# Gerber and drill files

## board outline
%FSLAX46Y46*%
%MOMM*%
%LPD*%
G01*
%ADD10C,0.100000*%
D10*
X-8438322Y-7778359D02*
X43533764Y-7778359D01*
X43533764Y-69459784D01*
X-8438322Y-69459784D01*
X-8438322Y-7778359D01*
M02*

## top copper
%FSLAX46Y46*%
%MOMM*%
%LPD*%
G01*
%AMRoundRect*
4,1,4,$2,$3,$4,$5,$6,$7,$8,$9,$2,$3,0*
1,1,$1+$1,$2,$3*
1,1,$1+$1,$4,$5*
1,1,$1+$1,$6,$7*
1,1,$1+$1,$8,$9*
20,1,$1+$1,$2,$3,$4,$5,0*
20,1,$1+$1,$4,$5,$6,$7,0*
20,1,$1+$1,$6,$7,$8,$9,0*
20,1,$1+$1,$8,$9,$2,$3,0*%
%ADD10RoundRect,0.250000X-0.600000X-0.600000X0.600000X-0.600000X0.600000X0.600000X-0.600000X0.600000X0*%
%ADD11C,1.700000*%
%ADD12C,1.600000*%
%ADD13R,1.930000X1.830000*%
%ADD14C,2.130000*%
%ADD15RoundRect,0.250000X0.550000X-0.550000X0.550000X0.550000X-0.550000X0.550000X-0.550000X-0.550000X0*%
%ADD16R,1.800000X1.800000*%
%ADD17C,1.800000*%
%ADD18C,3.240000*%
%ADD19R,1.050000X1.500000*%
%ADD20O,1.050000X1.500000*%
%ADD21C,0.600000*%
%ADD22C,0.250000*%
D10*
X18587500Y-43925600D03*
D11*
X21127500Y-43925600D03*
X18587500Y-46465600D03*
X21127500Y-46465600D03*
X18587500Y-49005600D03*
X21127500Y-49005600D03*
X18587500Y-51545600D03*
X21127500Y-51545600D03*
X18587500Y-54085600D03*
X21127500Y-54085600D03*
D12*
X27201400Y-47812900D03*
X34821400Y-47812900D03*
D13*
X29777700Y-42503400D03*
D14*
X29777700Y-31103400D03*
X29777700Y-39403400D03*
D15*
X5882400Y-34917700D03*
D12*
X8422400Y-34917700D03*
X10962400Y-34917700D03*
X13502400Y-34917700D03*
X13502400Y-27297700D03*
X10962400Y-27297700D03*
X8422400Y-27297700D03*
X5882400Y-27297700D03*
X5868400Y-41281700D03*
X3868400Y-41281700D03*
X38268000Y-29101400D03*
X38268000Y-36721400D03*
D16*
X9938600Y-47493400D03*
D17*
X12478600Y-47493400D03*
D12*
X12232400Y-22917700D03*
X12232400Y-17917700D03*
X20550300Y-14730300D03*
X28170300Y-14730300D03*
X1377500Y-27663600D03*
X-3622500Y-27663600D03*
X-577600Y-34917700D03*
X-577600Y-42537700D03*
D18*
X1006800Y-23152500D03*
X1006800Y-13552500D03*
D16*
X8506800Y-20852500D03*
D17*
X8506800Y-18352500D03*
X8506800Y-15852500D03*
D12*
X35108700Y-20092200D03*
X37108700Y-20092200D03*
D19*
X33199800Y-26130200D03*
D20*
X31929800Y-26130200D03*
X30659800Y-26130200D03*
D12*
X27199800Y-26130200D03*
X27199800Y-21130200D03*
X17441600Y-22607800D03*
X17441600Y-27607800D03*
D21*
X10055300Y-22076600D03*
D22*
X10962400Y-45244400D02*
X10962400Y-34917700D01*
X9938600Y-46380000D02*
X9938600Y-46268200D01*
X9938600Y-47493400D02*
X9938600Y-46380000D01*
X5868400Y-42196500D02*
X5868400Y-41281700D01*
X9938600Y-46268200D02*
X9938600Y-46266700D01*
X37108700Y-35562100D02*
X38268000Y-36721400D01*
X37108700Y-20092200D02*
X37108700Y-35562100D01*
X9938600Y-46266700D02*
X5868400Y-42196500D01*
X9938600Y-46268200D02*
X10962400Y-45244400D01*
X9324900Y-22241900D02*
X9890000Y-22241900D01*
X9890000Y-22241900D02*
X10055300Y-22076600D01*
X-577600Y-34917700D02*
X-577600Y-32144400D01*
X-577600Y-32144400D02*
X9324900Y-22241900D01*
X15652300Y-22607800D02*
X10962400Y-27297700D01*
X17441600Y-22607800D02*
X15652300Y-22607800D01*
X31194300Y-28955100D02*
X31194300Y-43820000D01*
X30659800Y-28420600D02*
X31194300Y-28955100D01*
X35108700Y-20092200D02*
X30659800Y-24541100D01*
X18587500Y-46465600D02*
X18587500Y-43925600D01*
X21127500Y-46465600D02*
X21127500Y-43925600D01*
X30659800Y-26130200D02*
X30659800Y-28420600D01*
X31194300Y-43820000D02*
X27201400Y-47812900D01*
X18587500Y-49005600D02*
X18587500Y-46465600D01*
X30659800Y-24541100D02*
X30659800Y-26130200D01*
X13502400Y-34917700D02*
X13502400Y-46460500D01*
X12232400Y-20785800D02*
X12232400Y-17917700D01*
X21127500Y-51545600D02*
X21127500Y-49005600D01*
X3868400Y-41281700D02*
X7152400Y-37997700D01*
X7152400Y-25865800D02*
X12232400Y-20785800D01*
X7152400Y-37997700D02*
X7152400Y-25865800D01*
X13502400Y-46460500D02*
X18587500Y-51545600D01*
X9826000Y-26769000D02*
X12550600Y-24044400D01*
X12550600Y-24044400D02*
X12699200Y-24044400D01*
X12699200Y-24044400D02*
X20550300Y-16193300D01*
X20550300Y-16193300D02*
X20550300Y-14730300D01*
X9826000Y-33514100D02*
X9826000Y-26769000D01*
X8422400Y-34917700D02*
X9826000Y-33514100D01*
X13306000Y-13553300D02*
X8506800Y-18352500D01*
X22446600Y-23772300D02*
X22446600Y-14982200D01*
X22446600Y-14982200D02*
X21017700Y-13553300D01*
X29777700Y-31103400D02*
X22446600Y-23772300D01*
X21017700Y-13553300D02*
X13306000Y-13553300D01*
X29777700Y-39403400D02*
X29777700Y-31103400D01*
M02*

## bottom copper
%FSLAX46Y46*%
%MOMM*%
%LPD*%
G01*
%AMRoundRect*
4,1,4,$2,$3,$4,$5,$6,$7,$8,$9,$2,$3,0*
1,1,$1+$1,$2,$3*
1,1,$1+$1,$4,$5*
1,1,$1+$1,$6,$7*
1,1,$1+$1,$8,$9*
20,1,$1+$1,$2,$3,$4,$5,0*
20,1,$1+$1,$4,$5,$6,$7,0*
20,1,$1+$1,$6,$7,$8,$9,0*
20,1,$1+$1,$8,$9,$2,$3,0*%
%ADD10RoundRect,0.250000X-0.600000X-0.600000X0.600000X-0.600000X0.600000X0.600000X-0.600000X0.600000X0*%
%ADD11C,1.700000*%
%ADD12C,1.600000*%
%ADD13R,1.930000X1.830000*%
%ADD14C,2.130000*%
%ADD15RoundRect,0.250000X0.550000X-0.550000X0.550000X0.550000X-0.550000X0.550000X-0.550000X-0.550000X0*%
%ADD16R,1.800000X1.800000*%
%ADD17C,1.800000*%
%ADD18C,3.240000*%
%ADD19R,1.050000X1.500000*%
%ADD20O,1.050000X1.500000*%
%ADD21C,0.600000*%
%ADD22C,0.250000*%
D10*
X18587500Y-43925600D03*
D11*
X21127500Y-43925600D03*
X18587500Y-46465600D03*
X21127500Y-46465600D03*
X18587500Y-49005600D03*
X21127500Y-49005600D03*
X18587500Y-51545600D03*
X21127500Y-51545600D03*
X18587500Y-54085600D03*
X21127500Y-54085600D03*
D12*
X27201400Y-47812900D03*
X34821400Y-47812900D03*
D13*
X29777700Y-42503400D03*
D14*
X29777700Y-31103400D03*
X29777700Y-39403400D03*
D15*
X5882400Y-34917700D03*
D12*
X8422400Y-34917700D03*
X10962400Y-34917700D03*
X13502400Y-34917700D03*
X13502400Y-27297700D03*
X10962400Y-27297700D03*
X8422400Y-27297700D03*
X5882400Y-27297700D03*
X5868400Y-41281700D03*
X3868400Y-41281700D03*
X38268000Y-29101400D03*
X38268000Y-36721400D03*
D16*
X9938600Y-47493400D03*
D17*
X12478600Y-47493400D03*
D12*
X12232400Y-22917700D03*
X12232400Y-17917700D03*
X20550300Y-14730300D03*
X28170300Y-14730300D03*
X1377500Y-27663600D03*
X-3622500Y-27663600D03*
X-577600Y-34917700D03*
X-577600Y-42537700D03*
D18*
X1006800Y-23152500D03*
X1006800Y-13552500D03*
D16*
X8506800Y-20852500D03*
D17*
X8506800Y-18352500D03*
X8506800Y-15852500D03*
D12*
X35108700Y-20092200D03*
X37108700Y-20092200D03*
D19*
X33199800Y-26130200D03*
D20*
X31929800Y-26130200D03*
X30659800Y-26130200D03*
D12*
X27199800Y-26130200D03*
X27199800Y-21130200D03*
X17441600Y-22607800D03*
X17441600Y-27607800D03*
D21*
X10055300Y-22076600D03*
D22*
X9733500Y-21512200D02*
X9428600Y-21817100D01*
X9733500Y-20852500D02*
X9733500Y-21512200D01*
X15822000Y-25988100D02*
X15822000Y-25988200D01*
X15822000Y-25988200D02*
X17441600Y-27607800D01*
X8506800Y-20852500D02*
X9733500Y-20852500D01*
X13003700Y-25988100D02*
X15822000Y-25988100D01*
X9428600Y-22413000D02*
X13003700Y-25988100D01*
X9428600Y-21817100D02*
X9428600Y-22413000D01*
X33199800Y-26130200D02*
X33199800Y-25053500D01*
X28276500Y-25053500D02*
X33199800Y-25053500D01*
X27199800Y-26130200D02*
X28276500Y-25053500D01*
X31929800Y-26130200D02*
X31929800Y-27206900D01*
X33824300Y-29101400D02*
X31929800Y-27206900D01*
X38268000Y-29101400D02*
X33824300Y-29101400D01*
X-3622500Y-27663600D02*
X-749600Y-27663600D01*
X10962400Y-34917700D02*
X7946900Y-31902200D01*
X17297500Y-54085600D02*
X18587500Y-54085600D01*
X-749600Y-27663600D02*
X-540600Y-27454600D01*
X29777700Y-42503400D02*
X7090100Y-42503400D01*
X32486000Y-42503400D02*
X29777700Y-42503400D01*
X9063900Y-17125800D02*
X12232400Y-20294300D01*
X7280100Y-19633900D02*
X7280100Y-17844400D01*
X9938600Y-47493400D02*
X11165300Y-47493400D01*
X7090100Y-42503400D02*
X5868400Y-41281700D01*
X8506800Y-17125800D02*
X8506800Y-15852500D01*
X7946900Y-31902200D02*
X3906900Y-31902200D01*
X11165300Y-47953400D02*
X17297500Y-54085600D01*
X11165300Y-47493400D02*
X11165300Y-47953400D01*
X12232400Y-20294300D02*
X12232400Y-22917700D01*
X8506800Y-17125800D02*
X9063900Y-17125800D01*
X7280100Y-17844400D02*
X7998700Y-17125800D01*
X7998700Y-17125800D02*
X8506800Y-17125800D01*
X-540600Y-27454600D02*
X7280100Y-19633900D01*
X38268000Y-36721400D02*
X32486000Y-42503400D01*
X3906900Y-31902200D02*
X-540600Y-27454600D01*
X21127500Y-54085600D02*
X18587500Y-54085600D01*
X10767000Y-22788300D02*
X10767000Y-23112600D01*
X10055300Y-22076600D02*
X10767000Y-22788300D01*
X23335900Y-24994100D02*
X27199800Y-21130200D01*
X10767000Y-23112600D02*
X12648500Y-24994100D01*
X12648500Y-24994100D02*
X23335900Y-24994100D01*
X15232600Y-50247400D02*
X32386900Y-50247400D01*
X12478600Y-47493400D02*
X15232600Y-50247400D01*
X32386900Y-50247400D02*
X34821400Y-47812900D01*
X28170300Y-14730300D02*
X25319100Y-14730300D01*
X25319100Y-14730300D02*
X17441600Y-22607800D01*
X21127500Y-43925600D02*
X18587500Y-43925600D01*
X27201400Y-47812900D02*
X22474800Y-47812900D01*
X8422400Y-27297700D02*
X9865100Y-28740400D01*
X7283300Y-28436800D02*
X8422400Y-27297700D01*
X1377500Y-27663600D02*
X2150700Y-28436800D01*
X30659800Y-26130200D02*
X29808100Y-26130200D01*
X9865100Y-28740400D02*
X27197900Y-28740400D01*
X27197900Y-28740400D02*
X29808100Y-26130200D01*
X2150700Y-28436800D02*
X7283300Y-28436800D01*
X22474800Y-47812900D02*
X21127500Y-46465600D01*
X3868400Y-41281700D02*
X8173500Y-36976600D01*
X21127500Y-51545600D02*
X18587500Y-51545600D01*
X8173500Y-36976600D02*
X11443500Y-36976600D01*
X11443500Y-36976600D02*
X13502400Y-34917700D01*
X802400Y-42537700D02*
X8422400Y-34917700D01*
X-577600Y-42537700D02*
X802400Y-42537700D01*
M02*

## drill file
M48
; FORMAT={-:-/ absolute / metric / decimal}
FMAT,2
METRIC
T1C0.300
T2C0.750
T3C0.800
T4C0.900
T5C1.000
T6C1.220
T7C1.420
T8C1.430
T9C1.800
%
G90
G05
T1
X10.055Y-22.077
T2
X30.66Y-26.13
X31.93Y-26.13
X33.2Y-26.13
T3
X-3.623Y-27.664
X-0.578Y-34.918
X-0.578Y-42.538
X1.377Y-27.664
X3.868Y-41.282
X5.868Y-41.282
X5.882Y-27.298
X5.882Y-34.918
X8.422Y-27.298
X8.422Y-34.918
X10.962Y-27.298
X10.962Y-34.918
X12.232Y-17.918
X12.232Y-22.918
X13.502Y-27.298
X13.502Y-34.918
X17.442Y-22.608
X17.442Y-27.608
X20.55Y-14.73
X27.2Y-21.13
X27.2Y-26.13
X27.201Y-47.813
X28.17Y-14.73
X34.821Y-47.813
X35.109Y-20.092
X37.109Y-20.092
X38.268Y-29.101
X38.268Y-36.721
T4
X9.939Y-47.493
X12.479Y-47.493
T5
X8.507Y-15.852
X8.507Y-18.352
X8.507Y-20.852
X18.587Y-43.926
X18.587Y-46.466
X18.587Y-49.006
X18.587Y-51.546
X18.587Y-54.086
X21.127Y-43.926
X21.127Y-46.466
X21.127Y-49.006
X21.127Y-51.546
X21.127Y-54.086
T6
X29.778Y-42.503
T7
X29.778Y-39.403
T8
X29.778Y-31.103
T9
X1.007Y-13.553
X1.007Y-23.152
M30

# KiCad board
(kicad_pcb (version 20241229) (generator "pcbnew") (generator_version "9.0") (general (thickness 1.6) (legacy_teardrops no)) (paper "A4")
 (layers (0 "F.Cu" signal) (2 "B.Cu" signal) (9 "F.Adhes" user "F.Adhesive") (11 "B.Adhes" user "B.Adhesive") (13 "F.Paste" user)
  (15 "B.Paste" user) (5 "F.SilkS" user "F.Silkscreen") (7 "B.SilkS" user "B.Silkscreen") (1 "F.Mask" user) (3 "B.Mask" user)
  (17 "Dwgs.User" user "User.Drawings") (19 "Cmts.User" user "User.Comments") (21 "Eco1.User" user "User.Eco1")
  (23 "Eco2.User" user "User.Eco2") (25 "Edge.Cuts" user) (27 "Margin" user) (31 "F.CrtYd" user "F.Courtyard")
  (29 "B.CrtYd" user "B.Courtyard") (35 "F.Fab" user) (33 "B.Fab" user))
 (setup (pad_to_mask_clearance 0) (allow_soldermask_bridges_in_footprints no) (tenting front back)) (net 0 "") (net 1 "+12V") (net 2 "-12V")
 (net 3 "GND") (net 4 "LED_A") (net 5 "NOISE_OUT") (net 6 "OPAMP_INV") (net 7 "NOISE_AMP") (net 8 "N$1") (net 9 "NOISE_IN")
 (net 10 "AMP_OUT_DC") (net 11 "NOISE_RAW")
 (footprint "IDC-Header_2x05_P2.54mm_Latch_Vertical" (layer "F.Cu") (at 18.5875 43.9256)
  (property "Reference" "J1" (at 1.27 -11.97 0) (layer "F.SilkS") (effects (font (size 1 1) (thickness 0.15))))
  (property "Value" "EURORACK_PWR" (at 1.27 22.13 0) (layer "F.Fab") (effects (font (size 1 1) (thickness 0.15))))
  (pad "1" thru_hole roundrect (at 0 0) (size 1.7 1.7) (drill 1) (layers "*.Cu" "*.Mask") (remove_unused_layers no)
   (roundrect_rratio 0.147059) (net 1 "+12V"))
  (pad "2" thru_hole circle (at 2.54 0) (size 1.7 1.7) (drill 1) (layers "*.Cu" "*.Mask") (remove_unused_layers no) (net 1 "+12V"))
  (pad "3" thru_hole circle (at 0 2.54) (size 1.7 1.7) (drill 1) (layers "*.Cu" "*.Mask") (remove_unused_layers no) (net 1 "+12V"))
  (pad "4" thru_hole circle (at 2.54 2.54) (size 1.7 1.7) (drill 1) (layers "*.Cu" "*.Mask") (remove_unused_layers no) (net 1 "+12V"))
  (pad "5" thru_hole circle (at 0 5.08) (size 1.7 1.7) (drill 1) (layers "*.Cu" "*.Mask") (remove_unused_layers no) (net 1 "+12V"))
  (pad "6" thru_hole circle (at 2.54 5.08) (size 1.7 1.7) (drill 1) (layers "*.Cu" "*.Mask") (remove_unused_layers no) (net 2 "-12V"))
  (pad "7" thru_hole circle (at 0 7.62) (size 1.7 1.7) (drill 1) (layers "*.Cu" "*.Mask") (remove_unused_layers no) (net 2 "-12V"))
  (pad "8" thru_hole circle (at 2.54 7.62) (size 1.7 1.7) (drill 1) (layers "*.Cu" "*.Mask") (remove_unused_layers no) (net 2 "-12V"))
  (pad "9" thru_hole circle (at 0 10.16) (size 1.7 1.7) (drill 1) (layers "*.Cu" "*.Mask") (remove_unused_layers no) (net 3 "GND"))
  (pad "10" thru_hole circle (at 2.54 10.16) (size 1.7 1.7) (drill 1) (layers "*.Cu" "*.Mask") (remove_unused_layers no) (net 3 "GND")))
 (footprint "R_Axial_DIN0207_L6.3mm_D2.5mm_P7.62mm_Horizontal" (layer "F.Cu") (at 27.2014 47.8129)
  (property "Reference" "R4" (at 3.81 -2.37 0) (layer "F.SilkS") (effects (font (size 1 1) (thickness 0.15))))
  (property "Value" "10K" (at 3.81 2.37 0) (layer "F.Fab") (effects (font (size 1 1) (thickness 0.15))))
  (pad "1" thru_hole circle (at 0 0) (size 1.6 1.6) (drill 0.8) (layers "*.Cu" "*.Mask") (remove_unused_layers no) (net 1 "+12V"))
  (pad "2" thru_hole circle (at 7.62 0) (size 1.6 1.6) (drill 0.8) (layers "*.Cu" "*.Mask") (remove_unused_layers no) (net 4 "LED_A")))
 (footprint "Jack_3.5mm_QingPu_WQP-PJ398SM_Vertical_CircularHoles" (layer "F.Cu") (at 29.7777 42.5034 180)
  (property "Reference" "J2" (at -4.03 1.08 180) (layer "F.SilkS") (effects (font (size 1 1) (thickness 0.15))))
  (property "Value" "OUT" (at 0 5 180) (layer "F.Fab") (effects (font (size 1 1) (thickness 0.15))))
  (pad "S" thru_hole rect (at 0 0) (size 1.93 1.83) (drill 1.22) (layers "*.Cu" "*.Mask") (remove_unused_layers no) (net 3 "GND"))
  (pad "T" thru_hole circle (at 0 11.4) (size 2.13 2.13) (drill 1.43) (layers "*.Cu" "*.Mask") (remove_unused_layers no) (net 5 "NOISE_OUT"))
  (pad "TN" thru_hole circle (at 0 3.1) (size 2.13 2.13) (drill 1.42) (layers "*.Cu" "*.Mask") (remove_unused_layers no) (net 5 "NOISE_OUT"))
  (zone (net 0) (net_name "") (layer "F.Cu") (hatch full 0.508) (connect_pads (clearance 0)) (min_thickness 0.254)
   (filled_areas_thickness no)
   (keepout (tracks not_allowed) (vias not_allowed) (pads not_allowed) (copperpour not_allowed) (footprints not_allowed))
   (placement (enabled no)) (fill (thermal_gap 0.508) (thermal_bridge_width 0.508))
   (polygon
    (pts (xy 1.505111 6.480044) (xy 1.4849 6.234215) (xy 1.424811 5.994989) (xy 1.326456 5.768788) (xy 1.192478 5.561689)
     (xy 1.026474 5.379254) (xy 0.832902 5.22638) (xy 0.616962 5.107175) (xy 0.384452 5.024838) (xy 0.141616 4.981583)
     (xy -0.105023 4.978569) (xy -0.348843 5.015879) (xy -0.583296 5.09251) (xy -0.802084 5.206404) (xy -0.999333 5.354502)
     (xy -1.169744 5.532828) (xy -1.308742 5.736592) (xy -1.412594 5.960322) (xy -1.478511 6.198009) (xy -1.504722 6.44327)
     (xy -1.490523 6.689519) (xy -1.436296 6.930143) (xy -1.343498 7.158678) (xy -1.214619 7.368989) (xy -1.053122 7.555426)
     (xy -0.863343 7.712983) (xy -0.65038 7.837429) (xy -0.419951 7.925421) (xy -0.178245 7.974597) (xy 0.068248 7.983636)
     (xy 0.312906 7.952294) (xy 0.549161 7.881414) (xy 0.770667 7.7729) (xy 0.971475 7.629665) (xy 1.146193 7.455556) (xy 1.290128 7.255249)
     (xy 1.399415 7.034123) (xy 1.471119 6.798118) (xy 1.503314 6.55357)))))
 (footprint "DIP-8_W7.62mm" (layer "F.Cu") (at 5.8824 34.9177 90)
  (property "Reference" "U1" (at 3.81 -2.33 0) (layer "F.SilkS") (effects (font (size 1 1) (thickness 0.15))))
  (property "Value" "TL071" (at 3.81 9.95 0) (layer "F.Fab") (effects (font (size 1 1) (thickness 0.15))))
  (pad "1" thru_hole roundrect (at 0 0 90) (size 1.6 1.6) (drill 0.8) (layers "*.Cu" "*.Mask") (remove_unused_layers no)
   (roundrect_rratio 0.15625))
  (pad "2" thru_hole circle (at 0 2.54 90) (size 1.6 1.6) (drill 0.8) (layers "*.Cu" "*.Mask") (remove_unused_layers no) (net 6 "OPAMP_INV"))
  (pad "3" thru_hole circle (at 0 5.08 90) (size 1.6 1.6) (drill 0.8) (layers "*.Cu" "*.Mask") (remove_unused_layers no) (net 3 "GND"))
  (pad "4" thru_hole circle (at 0 7.62 90) (size 1.6 1.6) (drill 0.8) (layers "*.Cu" "*.Mask") (remove_unused_layers no) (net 2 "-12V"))
  (pad "5" thru_hole circle (at 7.62 7.62 90) (size 1.6 1.6) (drill 0.8) (layers "*.Cu" "*.Mask") (remove_unused_layers no))
  (pad "6" thru_hole circle (at 7.62 5.08 90) (size 1.6 1.6) (drill 0.8) (layers "*.Cu" "*.Mask") (remove_unused_layers no)
   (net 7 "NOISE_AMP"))
  (pad "7" thru_hole circle (at 7.62 2.54 90) (size 1.6 1.6) (drill 0.8) (layers "*.Cu" "*.Mask") (remove_unused_layers no) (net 1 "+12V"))
  (pad "8" thru_hole circle (at 7.62 0 90) (size 1.6 1.6) (drill 0.8) (layers "*.Cu" "*.Mask") (remove_unused_layers no)))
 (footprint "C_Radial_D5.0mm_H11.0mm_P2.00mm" (layer "F.Cu") (at 5.8684 41.2817 180)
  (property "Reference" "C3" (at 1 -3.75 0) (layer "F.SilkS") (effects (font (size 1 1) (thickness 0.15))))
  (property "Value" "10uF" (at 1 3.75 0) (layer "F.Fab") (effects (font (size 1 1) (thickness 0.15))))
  (pad "1" thru_hole circle (at 0 0 180) (size 1.6 1.6) (drill 0.8) (layers "*.Cu" "*.Mask") (remove_unused_layers no) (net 3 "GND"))
  (pad "2" thru_hole circle (at 2 0 180) (size 1.6 1.6) (drill 0.8) (layers "*.Cu" "*.Mask") (remove_unused_layers no) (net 2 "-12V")))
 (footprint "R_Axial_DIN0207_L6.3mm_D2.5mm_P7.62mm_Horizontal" (layer "F.Cu") (at 38.268 29.1014 -90)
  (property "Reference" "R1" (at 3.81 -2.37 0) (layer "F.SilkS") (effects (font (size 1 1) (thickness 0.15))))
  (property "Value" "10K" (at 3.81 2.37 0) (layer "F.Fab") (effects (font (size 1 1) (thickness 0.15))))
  (pad "1" thru_hole circle (at 0 0 270) (size 1.6 1.6) (drill 0.8) (layers "*.Cu" "*.Mask") (remove_unused_layers no) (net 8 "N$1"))
  (pad "2" thru_hole circle (at 7.62 0 270) (size 1.6 1.6) (drill 0.8) (layers "*.Cu" "*.Mask") (remove_unused_layers no) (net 3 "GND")))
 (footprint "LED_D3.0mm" (layer "F.Cu") (at 9.9386 47.4934)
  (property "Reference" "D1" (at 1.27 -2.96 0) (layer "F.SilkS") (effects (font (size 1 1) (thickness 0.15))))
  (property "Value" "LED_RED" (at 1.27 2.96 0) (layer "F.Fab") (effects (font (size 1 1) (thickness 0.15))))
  (pad "1" thru_hole rect (at 0 0) (size 1.8 1.8) (drill 0.9) (layers "*.Cu" "*.Mask") (remove_unused_layers no) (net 3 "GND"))
  (pad "2" thru_hole circle (at 2.54 0) (size 1.8 1.8) (drill 0.9) (layers "*.Cu" "*.Mask") (remove_unused_layers no) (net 4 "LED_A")))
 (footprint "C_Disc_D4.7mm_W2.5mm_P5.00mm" (layer "F.Cu") (at 12.2324 22.9177 90)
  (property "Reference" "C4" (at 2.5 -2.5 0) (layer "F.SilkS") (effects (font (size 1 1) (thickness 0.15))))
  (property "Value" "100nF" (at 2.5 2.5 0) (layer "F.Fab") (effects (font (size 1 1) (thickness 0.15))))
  (pad "1" thru_hole circle (at 0 0 90) (size 1.6 1.6) (drill 0.8) (layers "*.Cu" "*.Mask") (remove_unused_layers no) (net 3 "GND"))
  (pad "2" thru_hole circle (at 5 0 90) (size 1.6 1.6) (drill 0.8) (layers "*.Cu" "*.Mask") (remove_unused_layers no) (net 2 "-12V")))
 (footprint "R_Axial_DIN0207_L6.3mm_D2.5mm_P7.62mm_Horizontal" (layer "F.Cu") (at 20.5503 14.7303)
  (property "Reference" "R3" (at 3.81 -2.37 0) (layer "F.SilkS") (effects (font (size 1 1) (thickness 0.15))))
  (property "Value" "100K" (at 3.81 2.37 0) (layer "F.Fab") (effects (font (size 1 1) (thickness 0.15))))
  (pad "1" thru_hole circle (at 0 0) (size 1.6 1.6) (drill 0.8) (layers "*.Cu" "*.Mask") (remove_unused_layers no) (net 6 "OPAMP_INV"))
  (pad "2" thru_hole circle (at 7.62 0) (size 1.6 1.6) (drill 0.8) (layers "*.Cu" "*.Mask") (remove_unused_layers no) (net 7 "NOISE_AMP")))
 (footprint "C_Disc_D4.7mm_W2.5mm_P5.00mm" (layer "F.Cu") (at 1.3775 27.6636 180)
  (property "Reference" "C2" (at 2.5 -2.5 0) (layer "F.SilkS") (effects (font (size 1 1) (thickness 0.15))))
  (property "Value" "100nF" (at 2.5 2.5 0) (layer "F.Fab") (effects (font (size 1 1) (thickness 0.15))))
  (pad "1" thru_hole circle (at 0 0 180) (size 1.6 1.6) (drill 0.8) (layers "*.Cu" "*.Mask") (remove_unused_layers no) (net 1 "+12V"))
  (pad "2" thru_hole circle (at 5 0 180) (size 1.6 1.6) (drill 0.8) (layers "*.Cu" "*.Mask") (remove_unused_layers no) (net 3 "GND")))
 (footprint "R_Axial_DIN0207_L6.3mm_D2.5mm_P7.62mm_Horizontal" (layer "F.Cu") (at -0.5776 34.9177 -90)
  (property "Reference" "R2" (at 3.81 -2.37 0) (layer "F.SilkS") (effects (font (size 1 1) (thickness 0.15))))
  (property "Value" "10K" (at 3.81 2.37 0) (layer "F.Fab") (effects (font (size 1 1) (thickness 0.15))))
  (pad "1" thru_hole circle (at 0 0 270) (size 1.6 1.6) (drill 0.8) (layers "*.Cu" "*.Mask") (remove_unused_layers no) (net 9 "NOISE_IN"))
  (pad "2" thru_hole circle (at 7.62 0 270) (size 1.6 1.6) (drill 0.8) (layers "*.Cu" "*.Mask") (remove_unused_layers no)
   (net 6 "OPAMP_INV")))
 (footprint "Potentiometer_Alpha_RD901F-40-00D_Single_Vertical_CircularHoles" (layer "F.Cu") (at 8.5068 20.8525 180)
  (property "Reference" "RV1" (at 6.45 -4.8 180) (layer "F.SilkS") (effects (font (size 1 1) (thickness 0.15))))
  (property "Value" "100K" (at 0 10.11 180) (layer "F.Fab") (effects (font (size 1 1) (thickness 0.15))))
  (pad "" thru_hole circle (at 7.5 -2.3 270) (size 3.24 3.24) (drill 1.8) (layers "*.Cu" "*.Mask") (remove_unused_layers no))
  (pad "" thru_hole circle (at 7.5 7.3 270) (size 3.24 3.24) (drill 1.8) (layers "*.Cu" "*.Mask") (remove_unused_layers no))
  (pad "1" thru_hole rect (at 0 0 270) (size 1.8 1.8) (drill 1) (layers "*.Cu" "*.Mask") (remove_unused_layers no) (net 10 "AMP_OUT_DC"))
  (pad "2" thru_hole circle (at 0 2.5 270) (size 1.8 1.8) (drill 1) (layers "*.Cu" "*.Mask") (remove_unused_layers no) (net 5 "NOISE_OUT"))
  (pad "3" thru_hole circle (at 0 5 270) (size 1.8 1.8) (drill 1) (layers "*.Cu" "*.Mask") (remove_unused_layers no) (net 3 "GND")))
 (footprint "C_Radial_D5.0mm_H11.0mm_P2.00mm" (layer "F.Cu") (at 35.1087 20.0922)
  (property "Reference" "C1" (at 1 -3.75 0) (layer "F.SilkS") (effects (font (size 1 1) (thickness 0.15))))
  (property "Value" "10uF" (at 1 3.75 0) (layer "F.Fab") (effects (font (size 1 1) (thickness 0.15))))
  (pad "1" thru_hole circle (at 0 0) (size 1.6 1.6) (drill 0.8) (layers "*.Cu" "*.Mask") (remove_unused_layers no) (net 1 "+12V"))
  (pad "2" thru_hole circle (at 2 0) (size 1.6 1.6) (drill 0.8) (layers "*.Cu" "*.Mask") (remove_unused_layers no) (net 3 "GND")))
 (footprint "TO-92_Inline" (layer "F.Cu") (at 33.1998 26.1302 180)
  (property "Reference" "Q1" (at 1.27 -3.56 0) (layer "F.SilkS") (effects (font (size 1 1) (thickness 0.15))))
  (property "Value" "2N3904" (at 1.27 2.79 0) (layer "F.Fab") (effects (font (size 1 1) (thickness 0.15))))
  (pad "1" thru_hole rect (at 0 0 180) (size 1.05 1.5) (drill 0.75) (layers "*.Cu" "*.Mask") (remove_unused_layers no) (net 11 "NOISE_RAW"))
  (pad "2" thru_hole oval (at 1.27 0 180) (size 1.05 1.5) (drill 0.75) (layers "*.Cu" "*.Mask") (remove_unused_layers no) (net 8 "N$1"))
  (pad "3" thru_hole oval (at 2.54 0 180) (size 1.05 1.5) (drill 0.75) (layers "*.Cu" "*.Mask") (remove_unused_layers no) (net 1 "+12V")))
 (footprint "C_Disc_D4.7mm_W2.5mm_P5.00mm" (layer "F.Cu") (at 27.1998 26.1302 90)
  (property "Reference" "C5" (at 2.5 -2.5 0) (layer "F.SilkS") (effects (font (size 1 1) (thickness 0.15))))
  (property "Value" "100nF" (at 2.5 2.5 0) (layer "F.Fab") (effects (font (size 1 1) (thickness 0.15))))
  (pad "1" thru_hole circle (at 0 0 90) (size 1.6 1.6) (drill 0.8) (layers "*.Cu" "*.Mask") (remove_unused_layers no) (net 11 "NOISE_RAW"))
  (pad "2" thru_hole circle (at 5 0 90) (size 1.6 1.6) (drill 0.8) (layers "*.Cu" "*.Mask") (remove_unused_layers no) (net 9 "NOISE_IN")))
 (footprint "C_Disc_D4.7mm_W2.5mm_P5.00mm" (layer "F.Cu") (at 17.4416 22.6078 -90)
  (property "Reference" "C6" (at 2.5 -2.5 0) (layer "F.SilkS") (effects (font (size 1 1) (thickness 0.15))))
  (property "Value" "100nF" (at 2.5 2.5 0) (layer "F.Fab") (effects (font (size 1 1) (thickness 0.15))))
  (pad "1" thru_hole circle (at 0 0 270) (size 1.6 1.6) (drill 0.8) (layers "*.Cu" "*.Mask") (remove_unused_layers no) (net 7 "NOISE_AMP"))
  (pad "2" thru_hole circle (at 5 0 270) (size 1.6 1.6) (drill 0.8) (layers "*.Cu" "*.Mask") (remove_unused_layers no) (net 10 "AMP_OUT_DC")))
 (gr_rect (start -8.438322 7.778359) (end 43.533764 69.459784) (stroke (width 0.1) (type solid)) (fill no) (layer "Edge.Cuts"))
 (segment (start 9.7335 21.5122) (end 9.4286 21.8171) (width 0.25) (layer "B.Cu") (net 10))
 (segment (start 9.7335 20.8525) (end 9.7335 21.5122) (width 0.25) (layer "B.Cu") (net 10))
 (segment (start 15.822 25.9881) (end 15.822 25.9882) (width 0.25) (layer "B.Cu") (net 10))
 (segment (start 15.822 25.9882) (end 17.4416 27.6078) (width 0.25) (layer "B.Cu") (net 10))
 (segment (start 8.5068 20.8525) (end 9.7335 20.8525) (width 0.25) (layer "B.Cu") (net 10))
 (segment (start 13.0037 25.9881) (end 15.822 25.9881) (width 0.25) (layer "B.Cu") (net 10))
 (segment (start 9.4286 22.413) (end 13.0037 25.9881) (width 0.25) (layer "B.Cu") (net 10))
 (segment (start 9.4286 21.8171) (end 9.4286 22.413) (width 0.25) (layer "B.Cu") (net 10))
 (segment (start 33.1998 26.1302) (end 33.1998 25.0535) (width 0.25) (layer "B.Cu") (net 11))
 (segment (start 28.2765 25.0535) (end 33.1998 25.0535) (width 0.25) (layer "B.Cu") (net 11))
 (segment (start 27.1998 26.1302) (end 28.2765 25.0535) (width 0.25) (layer "B.Cu") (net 11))
 (segment (start 31.9298 26.1302) (end 31.9298 27.2069) (width 0.25) (layer "B.Cu") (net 8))
 (segment (start 33.8243 29.1014) (end 31.9298 27.2069) (width 0.25) (layer "B.Cu") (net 8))
 (segment (start 38.268 29.1014) (end 33.8243 29.1014) (width 0.25) (layer "B.Cu") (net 8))
 (segment (start 10.9624 45.2444) (end 10.9624 34.9177) (width 0.25) (layer "F.Cu") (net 3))
 (segment (start 9.9386 46.38) (end 9.9386 46.2682) (width 0.25) (layer "F.Cu") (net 3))
 (segment (start 9.9386 47.4934) (end 9.9386 46.38) (width 0.25) (layer "F.Cu") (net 3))
 (segment (start 5.8684 42.1965) (end 5.8684 41.2817) (width 0.25) (layer "F.Cu") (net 3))
 (segment (start 9.9386 46.2682) (end 9.9386 46.2667) (width 0.25) (layer "F.Cu") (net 3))
 (segment (start 37.1087 35.5621) (end 38.268 36.7214) (width 0.25) (layer "F.Cu") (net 3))
 (segment (start 37.1087 20.0922) (end 37.1087 35.5621) (width 0.25) (layer "F.Cu") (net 3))
 (segment (start 9.9386 46.2667) (end 5.8684 42.1965) (width 0.25) (layer "F.Cu") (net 3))
 (segment (start 9.9386 46.2682) (end 10.9624 45.2444) (width 0.25) (layer "F.Cu") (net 3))
 (segment (start -3.6225 27.6636) (end -0.7496 27.6636) (width 0.25) (layer "B.Cu") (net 3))
 (segment (start 10.9624 34.9177) (end 7.9469 31.9022) (width 0.25) (layer "B.Cu") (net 3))
 (segment (start 17.2975 54.0856) (end 18.5875 54.0856) (width 0.25) (layer "B.Cu") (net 3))
 (segment (start -0.7496 27.6636) (end -0.5406 27.4546) (width 0.25) (layer "B.Cu") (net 3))
 (segment (start 29.7777 42.5034) (end 7.0901 42.5034) (width 0.25) (layer "B.Cu") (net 3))
 (segment (start 32.486 42.5034) (end 29.7777 42.5034) (width 0.25) (layer "B.Cu") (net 3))
 (segment (start 9.0639 17.1258) (end 12.2324 20.2943) (width 0.25) (layer "B.Cu") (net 3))
 (segment (start 7.2801 19.6339) (end 7.2801 17.8444) (width 0.25) (layer "B.Cu") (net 3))
 (segment (start 9.9386 47.4934) (end 11.1653 47.4934) (width 0.25) (layer "B.Cu") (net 3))
 (segment (start 7.0901 42.5034) (end 5.8684 41.2817) (width 0.25) (layer "B.Cu") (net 3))
 (segment (start 8.5068 17.1258) (end 8.5068 15.8525) (width 0.25) (layer "B.Cu") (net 3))
 (segment (start 7.9469 31.9022) (end 3.9069 31.9022) (width 0.25) (layer "B.Cu") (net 3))
 (segment (start 11.1653 47.9534) (end 17.2975 54.0856) (width 0.25) (layer "B.Cu") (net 3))
 (segment (start 11.1653 47.4934) (end 11.1653 47.9534) (width 0.25) (layer "B.Cu") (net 3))
 (segment (start 12.2324 20.2943) (end 12.2324 22.9177) (width 0.25) (layer "B.Cu") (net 3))
 (segment (start 8.5068 17.1258) (end 9.0639 17.1258) (width 0.25) (layer "B.Cu") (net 3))
 (segment (start 7.2801 17.8444) (end 7.9987 17.1258) (width 0.25) (layer "B.Cu") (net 3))
 (segment (start 7.9987 17.1258) (end 8.5068 17.1258) (width 0.25) (layer "B.Cu") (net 3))
 (segment (start -0.5406 27.4546) (end 7.2801 19.6339) (width 0.25) (layer "B.Cu") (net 3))
 (segment (start 38.268 36.7214) (end 32.486 42.5034) (width 0.25) (layer "B.Cu") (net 3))
 (segment (start 3.9069 31.9022) (end -0.5406 27.4546) (width 0.25) (layer "B.Cu") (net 3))
 (segment (start 21.1275 54.0856) (end 18.5875 54.0856) (width 0.25) (layer "B.Cu") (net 3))
 (segment (start 9.3249 22.2419) (end 9.89 22.2419) (width 0.25) (layer "F.Cu") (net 9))
 (segment (start 9.89 22.2419) (end 10.0553 22.0766) (width 0.25) (layer "F.Cu") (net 9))
 (segment (start -0.5776 34.9177) (end -0.5776 32.1444) (width 0.25) (layer "F.Cu") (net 9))
 (segment (start -0.5776 32.1444) (end 9.3249 22.2419) (width 0.25) (layer "F.Cu") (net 9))
 (via (at 10.0553 22.0766) (size 0.6) (drill 0.3) (layers "F.Cu" "B.Cu") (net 9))
 (segment (start 10.767 22.7883) (end 10.767 23.1126) (width 0.25) (layer "B.Cu") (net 9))
 (segment (start 10.0553 22.0766) (end 10.767 22.7883) (width 0.25) (layer "B.Cu") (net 9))
 (segment (start 23.3359 24.9941) (end 27.1998 21.1302) (width 0.25) (layer "B.Cu") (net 9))
 (segment (start 10.767 23.1126) (end 12.6485 24.9941) (width 0.25) (layer "B.Cu") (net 9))
 (segment (start 12.6485 24.9941) (end 23.3359 24.9941) (width 0.25) (layer "B.Cu") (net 9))
 (segment (start 15.2326 50.2474) (end 32.3869 50.2474) (width 0.25) (layer "B.Cu") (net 4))
 (segment (start 12.4786 47.4934) (end 15.2326 50.2474) (width 0.25) (layer "B.Cu") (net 4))
 (segment (start 32.3869 50.2474) (end 34.8214 47.8129) (width 0.25) (layer "B.Cu") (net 4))
 (segment (start 15.6523 22.6078) (end 10.9624 27.2977) (width 0.25) (layer "F.Cu") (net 7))
 (segment (start 17.4416 22.6078) (end 15.6523 22.6078) (width 0.25) (layer "F.Cu") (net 7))
 (segment (start 28.1703 14.7303) (end 25.3191 14.7303) (width 0.25) (layer "B.Cu") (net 7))
 (segment (start 25.3191 14.7303) (end 17.4416 22.6078) (width 0.25) (layer "B.Cu") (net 7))
 (segment (start 31.1943 28.9551) (end 31.1943 43.82) (width 0.25) (layer "F.Cu") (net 1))
 (segment (start 30.6598 28.4206) (end 31.1943 28.9551) (width 0.25) (layer "F.Cu") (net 1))
 (segment (start 35.1087 20.0922) (end 30.6598 24.5411) (width 0.25) (layer "F.Cu") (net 1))
 (segment (start 18.5875 46.4656) (end 18.5875 43.9256) (width 0.25) (layer "F.Cu") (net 1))
 (segment (start 21.1275 46.4656) (end 21.1275 43.9256) (width 0.25) (layer "F.Cu") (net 1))
 (segment (start 30.6598 26.1302) (end 30.6598 28.4206) (width 0.25) (layer "F.Cu") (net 1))
 (segment (start 31.1943 43.82) (end 27.2014 47.8129) (width 0.25) (layer "F.Cu") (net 1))
 (segment (start 18.5875 49.0056) (end 18.5875 46.4656) (width 0.25) (layer "F.Cu") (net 1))
 (segment (start 30.6598 24.5411) (end 30.6598 26.1302) (width 0.25) (layer "F.Cu") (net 1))
 (segment (start 21.1275 43.9256) (end 18.5875 43.9256) (width 0.25) (layer "B.Cu") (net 1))
 (segment (start 27.2014 47.8129) (end 22.4748 47.8129) (width 0.25) (layer "B.Cu") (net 1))
 (segment (start 8.4224 27.2977) (end 9.8651 28.7404) (width 0.25) (layer "B.Cu") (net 1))
 (segment (start 7.2833 28.4368) (end 8.4224 27.2977) (width 0.25) (layer "B.Cu") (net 1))
 (segment (start 1.3775 27.6636) (end 2.1507 28.4368) (width 0.25) (layer "B.Cu") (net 1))
 (segment (start 30.6598 26.1302) (end 29.8081 26.1302) (width 0.25) (layer "B.Cu") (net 1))
 (segment (start 9.8651 28.7404) (end 27.1979 28.7404) (width 0.25) (layer "B.Cu") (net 1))
 (segment (start 27.1979 28.7404) (end 29.8081 26.1302) (width 0.25) (layer "B.Cu") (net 1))
 (segment (start 2.1507 28.4368) (end 7.2833 28.4368) (width 0.25) (layer "B.Cu") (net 1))
 (segment (start 22.4748 47.8129) (end 21.1275 46.4656) (width 0.25) (layer "B.Cu") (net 1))
 (segment (start 13.5024 34.9177) (end 13.5024 46.4605) (width 0.25) (layer "F.Cu") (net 2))
 (segment (start 12.2324 20.7858) (end 12.2324 17.9177) (width 0.25) (layer "F.Cu") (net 2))
 (segment (start 21.1275 51.5456) (end 21.1275 49.0056) (width 0.25) (layer "F.Cu") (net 2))
 (segment (start 3.8684 41.2817) (end 7.1524 37.9977) (width 0.25) (layer "F.Cu") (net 2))
 (segment (start 7.1524 25.8658) (end 12.2324 20.7858) (width 0.25) (layer "F.Cu") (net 2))
 (segment (start 7.1524 37.9977) (end 7.1524 25.8658) (width 0.25) (layer "F.Cu") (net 2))
 (segment (start 13.5024 46.4605) (end 18.5875 51.5456) (width 0.25) (layer "F.Cu") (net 2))
 (segment (start 3.8684 41.2817) (end 8.1735 36.9766) (width 0.25) (layer "B.Cu") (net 2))
 (segment (start 21.1275 51.5456) (end 18.5875 51.5456) (width 0.25) (layer "B.Cu") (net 2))
 (segment (start 8.1735 36.9766) (end 11.4435 36.9766) (width 0.25) (layer "B.Cu") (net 2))
 (segment (start 11.4435 36.9766) (end 13.5024 34.9177) (width 0.25) (layer "B.Cu") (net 2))
 (segment (start 9.826 26.769) (end 12.5506 24.0444) (width 0.25) (layer "F.Cu") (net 6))
 (segment (start 12.5506 24.0444) (end 12.6992 24.0444) (width 0.25) (layer "F.Cu") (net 6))
 (segment (start 12.6992 24.0444) (end 20.5503 16.1933) (width 0.25) (layer "F.Cu") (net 6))
 (segment (start 20.5503 16.1933) (end 20.5503 14.7303) (width 0.25) (layer "F.Cu") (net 6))
 (segment (start 9.826 33.5141) (end 9.826 26.769) (width 0.25) (layer "F.Cu") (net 6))
 (segment (start 8.4224 34.9177) (end 9.826 33.5141) (width 0.25) (layer "F.Cu") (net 6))
 (segment (start 0.8024 42.5377) (end 8.4224 34.9177) (width 0.25) (layer "B.Cu") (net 6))
 (segment (start -0.5776 42.5377) (end 0.8024 42.5377) (width 0.25) (layer "B.Cu") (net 6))
 (segment (start 13.306 13.5533) (end 8.5068 18.3525) (width 0.25) (layer "F.Cu") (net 5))
 (segment (start 22.4466 23.7723) (end 22.4466 14.9822) (width 0.25) (layer "F.Cu") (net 5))
 (segment (start 22.4466 14.9822) (end 21.0177 13.5533) (width 0.25) (layer "F.Cu") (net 5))
 (segment (start 29.7777 31.1034) (end 22.4466 23.7723) (width 0.25) (layer "F.Cu") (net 5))
 (segment (start 21.0177 13.5533) (end 13.306 13.5533) (width 0.25) (layer "F.Cu") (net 5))
 (segment (start 29.7777 39.4034) (end 29.7777 31.1034) (width 0.25) (layer "F.Cu") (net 5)))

